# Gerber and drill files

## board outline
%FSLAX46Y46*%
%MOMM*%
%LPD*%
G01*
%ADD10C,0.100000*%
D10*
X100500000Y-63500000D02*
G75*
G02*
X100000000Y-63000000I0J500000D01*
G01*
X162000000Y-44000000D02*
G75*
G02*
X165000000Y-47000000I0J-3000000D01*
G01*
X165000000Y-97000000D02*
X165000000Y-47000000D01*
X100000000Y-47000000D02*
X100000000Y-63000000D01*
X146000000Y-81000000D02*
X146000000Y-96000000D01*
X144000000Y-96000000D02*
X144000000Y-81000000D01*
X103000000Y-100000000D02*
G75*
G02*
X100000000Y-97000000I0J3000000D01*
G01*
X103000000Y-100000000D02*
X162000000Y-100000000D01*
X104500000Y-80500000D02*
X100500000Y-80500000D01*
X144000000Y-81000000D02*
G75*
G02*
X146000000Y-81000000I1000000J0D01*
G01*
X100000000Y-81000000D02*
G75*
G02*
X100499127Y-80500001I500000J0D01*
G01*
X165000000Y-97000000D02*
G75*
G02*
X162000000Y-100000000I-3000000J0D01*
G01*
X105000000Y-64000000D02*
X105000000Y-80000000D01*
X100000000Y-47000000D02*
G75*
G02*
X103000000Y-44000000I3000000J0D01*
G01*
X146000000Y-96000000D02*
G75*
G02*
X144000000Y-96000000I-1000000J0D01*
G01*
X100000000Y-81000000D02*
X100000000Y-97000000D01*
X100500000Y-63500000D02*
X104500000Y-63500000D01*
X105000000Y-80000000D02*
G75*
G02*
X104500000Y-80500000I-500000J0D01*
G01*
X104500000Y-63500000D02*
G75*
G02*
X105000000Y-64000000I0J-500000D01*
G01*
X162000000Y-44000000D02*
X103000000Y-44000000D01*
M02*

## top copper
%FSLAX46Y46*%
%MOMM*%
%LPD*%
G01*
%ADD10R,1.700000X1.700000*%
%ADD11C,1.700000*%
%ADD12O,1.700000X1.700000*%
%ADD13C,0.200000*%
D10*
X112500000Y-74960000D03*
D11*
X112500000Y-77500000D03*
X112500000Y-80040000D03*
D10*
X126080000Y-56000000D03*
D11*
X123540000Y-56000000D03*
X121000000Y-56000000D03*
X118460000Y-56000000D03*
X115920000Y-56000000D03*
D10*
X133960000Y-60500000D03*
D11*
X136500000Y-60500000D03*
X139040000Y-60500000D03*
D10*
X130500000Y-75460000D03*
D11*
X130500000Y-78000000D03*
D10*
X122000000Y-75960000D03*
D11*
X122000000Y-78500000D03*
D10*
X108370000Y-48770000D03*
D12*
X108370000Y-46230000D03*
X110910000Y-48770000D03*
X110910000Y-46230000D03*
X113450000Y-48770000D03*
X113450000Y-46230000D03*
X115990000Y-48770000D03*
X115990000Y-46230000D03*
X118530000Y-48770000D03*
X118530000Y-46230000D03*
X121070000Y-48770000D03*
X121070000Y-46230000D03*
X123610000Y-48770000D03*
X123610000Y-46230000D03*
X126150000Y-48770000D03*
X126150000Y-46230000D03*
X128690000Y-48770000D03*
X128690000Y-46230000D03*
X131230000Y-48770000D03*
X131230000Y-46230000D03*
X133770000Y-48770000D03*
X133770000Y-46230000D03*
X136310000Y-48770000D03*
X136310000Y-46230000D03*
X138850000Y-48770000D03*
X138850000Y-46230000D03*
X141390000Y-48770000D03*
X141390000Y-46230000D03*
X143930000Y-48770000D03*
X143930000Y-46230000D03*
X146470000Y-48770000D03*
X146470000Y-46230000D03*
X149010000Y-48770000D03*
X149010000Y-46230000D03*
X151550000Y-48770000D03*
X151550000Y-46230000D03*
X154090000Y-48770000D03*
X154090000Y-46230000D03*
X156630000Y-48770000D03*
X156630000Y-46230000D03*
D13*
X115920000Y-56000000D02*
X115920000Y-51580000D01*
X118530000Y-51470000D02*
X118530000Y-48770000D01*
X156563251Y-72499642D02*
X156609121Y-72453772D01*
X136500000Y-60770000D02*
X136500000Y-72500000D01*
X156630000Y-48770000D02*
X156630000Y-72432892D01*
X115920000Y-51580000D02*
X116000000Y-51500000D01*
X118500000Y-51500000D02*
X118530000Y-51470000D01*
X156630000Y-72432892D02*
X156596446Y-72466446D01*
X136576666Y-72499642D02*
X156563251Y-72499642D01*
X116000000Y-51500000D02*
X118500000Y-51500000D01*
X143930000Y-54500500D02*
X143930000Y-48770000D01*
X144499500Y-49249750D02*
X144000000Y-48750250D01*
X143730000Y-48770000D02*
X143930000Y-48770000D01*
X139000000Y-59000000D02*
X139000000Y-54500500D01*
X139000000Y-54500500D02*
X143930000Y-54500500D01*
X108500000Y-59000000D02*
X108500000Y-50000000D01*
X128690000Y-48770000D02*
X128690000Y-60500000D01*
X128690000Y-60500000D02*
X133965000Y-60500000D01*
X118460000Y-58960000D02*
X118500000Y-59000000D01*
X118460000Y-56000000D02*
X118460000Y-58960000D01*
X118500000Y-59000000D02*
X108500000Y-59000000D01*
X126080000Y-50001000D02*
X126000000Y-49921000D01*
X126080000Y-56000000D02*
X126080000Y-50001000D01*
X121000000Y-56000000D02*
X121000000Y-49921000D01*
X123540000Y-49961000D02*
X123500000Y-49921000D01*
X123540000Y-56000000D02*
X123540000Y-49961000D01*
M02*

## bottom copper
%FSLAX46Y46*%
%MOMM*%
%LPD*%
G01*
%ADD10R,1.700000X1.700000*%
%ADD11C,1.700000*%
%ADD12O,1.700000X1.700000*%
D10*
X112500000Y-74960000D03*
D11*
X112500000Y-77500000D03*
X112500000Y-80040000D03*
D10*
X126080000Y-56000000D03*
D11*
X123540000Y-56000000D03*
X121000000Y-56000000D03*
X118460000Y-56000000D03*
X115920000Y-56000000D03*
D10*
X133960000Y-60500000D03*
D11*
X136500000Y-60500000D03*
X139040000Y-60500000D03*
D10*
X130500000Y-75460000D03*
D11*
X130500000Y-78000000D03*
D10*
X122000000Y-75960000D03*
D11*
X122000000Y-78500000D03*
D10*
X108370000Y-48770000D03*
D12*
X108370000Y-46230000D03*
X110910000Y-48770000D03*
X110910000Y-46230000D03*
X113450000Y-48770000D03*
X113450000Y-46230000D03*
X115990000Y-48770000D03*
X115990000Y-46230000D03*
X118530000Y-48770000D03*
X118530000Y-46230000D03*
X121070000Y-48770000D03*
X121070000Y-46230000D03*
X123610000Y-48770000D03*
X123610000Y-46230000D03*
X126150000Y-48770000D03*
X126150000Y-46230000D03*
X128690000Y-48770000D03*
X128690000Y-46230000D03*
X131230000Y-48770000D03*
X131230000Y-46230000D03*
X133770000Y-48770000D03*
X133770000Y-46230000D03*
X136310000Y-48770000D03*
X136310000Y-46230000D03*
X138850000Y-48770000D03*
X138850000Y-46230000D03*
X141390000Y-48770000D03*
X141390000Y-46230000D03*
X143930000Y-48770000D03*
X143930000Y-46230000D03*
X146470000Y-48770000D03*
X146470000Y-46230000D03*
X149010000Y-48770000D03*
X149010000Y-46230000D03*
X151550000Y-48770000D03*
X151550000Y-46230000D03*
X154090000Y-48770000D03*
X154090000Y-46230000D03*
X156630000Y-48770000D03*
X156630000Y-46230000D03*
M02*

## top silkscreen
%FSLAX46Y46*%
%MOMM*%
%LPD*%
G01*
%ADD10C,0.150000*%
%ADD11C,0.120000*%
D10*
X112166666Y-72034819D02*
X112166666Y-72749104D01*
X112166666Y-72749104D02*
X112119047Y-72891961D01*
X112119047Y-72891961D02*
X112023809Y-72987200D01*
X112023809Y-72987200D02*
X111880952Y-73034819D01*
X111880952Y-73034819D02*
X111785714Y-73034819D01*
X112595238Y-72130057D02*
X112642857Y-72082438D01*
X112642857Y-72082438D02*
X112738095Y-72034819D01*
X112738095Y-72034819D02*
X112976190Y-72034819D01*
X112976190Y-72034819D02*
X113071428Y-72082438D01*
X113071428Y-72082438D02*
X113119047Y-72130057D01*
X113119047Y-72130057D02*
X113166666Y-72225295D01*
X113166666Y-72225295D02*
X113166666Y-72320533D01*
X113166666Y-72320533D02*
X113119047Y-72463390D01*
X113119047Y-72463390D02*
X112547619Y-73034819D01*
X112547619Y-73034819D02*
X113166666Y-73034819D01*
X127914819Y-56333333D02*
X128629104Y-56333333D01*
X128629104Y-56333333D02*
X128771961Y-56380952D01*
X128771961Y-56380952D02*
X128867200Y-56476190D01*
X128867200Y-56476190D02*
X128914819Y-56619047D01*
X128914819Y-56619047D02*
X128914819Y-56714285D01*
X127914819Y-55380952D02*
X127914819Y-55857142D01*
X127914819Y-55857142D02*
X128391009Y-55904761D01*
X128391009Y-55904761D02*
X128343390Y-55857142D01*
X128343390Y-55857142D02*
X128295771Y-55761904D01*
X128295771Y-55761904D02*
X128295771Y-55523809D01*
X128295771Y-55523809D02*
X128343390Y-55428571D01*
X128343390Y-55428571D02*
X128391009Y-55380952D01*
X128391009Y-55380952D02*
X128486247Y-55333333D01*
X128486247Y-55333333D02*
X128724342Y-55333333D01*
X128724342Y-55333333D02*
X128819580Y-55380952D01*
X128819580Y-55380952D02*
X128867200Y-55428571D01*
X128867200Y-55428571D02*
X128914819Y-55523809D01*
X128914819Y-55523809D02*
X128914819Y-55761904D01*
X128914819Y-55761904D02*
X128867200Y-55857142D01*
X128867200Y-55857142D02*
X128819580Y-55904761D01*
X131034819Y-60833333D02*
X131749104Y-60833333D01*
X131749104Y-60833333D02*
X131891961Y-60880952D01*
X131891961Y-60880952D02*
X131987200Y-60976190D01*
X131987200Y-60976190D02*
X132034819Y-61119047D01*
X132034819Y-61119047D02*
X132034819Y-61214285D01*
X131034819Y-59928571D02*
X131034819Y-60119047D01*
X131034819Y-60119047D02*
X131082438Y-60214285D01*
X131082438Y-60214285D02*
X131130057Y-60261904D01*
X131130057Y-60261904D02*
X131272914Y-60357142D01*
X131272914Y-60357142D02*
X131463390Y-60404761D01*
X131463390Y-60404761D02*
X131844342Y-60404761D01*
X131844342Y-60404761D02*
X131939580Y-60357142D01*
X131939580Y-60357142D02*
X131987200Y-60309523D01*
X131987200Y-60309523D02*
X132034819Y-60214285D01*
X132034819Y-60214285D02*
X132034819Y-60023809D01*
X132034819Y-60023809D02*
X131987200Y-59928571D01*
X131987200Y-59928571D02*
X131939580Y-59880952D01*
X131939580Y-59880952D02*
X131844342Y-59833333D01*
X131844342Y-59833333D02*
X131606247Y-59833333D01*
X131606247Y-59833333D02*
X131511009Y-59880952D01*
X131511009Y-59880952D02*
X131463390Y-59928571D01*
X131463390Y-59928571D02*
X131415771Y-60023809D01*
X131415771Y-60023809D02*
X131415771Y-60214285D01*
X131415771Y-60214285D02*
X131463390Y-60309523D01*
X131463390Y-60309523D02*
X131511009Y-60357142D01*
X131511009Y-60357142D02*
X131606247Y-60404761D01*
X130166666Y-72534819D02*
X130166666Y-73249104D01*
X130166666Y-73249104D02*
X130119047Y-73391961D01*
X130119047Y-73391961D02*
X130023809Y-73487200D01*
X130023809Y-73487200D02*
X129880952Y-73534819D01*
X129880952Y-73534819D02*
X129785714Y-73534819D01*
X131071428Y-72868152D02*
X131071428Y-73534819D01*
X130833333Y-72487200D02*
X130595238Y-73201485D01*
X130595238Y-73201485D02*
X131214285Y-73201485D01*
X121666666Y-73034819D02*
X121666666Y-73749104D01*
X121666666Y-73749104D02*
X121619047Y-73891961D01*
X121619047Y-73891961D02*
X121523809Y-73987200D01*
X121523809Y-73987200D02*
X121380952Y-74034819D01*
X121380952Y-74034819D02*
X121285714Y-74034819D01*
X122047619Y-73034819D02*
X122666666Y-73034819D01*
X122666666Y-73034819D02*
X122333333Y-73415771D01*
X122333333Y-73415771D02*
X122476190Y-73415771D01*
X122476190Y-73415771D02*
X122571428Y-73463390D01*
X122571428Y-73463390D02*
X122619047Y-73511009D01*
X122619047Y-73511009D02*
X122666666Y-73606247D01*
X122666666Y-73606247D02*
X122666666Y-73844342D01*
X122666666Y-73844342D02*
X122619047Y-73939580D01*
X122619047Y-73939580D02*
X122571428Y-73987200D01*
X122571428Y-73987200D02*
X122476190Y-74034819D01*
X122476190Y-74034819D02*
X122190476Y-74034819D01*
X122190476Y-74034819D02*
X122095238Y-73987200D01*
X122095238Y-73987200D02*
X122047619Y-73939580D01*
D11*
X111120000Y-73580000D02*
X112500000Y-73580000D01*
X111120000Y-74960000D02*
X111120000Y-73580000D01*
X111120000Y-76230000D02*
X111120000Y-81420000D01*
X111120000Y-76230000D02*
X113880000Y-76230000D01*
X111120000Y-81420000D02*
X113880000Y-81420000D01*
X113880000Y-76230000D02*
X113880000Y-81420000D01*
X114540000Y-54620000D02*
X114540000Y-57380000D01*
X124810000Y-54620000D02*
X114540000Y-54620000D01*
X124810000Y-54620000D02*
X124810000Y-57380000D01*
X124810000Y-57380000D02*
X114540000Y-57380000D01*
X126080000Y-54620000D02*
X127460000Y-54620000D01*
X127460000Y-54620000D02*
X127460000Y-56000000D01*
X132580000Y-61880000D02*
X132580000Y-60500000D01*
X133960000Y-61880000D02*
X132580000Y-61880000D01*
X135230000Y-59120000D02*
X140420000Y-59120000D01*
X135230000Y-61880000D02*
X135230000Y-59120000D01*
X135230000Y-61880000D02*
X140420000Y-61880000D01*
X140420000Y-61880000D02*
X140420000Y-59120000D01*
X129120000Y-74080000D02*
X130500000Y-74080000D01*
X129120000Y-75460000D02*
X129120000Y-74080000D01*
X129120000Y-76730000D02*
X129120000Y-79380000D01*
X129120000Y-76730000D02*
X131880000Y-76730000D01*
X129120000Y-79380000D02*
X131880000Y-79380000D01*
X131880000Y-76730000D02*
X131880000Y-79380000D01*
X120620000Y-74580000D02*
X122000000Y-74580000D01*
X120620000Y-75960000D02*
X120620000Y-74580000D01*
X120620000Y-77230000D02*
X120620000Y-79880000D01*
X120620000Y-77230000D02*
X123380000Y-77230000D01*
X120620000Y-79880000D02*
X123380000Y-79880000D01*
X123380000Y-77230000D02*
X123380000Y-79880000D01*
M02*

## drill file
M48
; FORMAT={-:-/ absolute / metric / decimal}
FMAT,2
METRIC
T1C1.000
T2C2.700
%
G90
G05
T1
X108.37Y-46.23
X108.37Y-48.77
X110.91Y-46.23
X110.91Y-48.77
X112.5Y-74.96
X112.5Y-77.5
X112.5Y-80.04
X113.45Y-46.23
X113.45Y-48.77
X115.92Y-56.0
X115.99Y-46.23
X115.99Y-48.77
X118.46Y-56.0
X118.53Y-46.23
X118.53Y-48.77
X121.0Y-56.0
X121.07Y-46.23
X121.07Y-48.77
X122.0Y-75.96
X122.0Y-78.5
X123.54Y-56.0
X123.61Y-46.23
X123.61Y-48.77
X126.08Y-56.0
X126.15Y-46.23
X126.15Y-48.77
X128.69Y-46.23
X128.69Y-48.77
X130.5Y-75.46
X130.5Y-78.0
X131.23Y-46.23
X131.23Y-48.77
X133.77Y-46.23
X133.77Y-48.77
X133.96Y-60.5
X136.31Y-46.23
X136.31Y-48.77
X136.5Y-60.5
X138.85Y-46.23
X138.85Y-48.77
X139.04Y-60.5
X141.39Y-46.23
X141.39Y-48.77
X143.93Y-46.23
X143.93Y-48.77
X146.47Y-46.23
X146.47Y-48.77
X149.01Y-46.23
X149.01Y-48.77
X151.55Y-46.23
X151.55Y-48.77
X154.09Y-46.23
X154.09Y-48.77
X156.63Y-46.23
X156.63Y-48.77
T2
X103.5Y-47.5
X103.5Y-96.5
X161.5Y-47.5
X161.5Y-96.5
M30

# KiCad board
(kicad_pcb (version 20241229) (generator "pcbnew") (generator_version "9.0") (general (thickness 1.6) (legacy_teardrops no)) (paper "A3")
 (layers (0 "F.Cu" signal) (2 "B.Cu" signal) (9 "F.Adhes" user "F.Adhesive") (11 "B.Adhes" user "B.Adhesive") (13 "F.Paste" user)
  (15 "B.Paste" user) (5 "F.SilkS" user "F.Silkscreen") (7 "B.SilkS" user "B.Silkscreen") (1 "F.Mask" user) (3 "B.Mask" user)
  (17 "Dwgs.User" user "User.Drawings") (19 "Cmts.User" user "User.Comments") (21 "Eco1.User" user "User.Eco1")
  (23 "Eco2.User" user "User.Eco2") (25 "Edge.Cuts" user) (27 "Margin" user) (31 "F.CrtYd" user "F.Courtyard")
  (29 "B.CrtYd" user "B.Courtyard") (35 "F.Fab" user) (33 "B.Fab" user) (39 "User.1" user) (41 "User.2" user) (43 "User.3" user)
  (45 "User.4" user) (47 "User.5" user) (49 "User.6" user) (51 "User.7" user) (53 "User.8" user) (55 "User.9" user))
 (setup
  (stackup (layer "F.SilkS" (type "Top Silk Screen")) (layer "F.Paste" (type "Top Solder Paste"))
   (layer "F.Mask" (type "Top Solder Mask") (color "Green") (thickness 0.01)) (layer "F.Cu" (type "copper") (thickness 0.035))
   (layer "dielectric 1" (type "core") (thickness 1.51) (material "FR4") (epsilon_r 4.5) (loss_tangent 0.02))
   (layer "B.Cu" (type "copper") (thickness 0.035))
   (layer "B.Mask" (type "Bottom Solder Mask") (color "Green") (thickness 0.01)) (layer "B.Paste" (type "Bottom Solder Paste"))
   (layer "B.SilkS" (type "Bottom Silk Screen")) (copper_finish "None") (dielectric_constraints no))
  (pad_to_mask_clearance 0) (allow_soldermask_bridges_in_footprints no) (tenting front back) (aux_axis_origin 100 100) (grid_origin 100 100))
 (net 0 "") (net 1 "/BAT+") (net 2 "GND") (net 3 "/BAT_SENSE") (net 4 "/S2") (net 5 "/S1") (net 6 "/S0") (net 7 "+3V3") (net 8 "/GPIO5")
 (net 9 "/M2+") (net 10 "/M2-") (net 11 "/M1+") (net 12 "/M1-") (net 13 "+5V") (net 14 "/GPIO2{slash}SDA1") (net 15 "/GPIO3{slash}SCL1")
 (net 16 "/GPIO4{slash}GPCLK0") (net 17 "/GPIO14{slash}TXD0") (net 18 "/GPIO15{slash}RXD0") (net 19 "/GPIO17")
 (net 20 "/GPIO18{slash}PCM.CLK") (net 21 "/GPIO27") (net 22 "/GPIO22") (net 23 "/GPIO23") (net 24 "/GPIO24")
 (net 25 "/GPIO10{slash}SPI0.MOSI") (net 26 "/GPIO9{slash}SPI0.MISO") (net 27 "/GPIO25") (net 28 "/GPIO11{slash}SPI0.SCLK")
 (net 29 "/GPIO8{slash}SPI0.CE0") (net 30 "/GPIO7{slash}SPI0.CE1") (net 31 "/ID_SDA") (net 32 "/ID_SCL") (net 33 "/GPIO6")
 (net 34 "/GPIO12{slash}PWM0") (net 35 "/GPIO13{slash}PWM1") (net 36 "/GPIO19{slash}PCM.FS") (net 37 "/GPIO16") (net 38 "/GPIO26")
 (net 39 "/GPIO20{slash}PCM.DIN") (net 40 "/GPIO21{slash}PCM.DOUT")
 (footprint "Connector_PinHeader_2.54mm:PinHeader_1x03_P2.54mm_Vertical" (layer "F.Cu") (at 112.5 74.96)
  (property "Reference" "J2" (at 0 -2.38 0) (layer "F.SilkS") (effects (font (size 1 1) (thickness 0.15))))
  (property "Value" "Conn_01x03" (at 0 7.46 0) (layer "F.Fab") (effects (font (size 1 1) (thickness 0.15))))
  (fp_line (start -1.38 -1.38) (end 0 -1.38) (stroke (width 0.12) (type solid)) (layer "F.SilkS"))
  (fp_line (start -1.38 0) (end -1.38 -1.38) (stroke (width 0.12) (type solid)) (layer "F.SilkS"))
  (fp_line (start -1.38 1.27) (end -1.38 6.46) (stroke (width 0.12) (type solid)) (layer "F.SilkS"))
  (fp_line (start -1.38 1.27) (end 1.38 1.27) (stroke (width 0.12) (type solid)) (layer "F.SilkS"))
  (fp_line (start -1.38 6.46) (end 1.38 6.46) (stroke (width 0.12) (type solid)) (layer "F.SilkS"))
  (fp_line (start 1.38 1.27) (end 1.38 6.46) (stroke (width 0.12) (type solid)) (layer "F.SilkS"))
  (pad "1" thru_hole rect (at 0 0) (size 1.7 1.7) (drill 1) (layers "*.Cu" "*.Mask") (remove_unused_layers no) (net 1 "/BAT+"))
  (pad "2" thru_hole circle (at 0 2.54) (size 1.7 1.7) (drill 1) (layers "*.Cu" "*.Mask") (remove_unused_layers no) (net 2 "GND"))
  (pad "3" thru_hole circle (at 0 5.08) (size 1.7 1.7) (drill 1) (layers "*.Cu" "*.Mask") (remove_unused_layers no) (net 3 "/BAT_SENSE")))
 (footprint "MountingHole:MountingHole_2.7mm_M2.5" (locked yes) (layer "F.Cu") (at 161.5 47.5)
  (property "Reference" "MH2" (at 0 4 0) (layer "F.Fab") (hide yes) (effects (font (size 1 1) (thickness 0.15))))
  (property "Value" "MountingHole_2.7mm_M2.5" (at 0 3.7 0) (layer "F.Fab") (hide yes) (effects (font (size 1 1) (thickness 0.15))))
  (pad "" np_thru_hole circle (at 0 0) (size 2.7 2.7) (drill 2.7) (layers "*.Cu" "*.Mask")))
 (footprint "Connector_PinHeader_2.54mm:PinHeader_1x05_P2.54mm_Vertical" (layer "F.Cu") (at 126.08 56 -90)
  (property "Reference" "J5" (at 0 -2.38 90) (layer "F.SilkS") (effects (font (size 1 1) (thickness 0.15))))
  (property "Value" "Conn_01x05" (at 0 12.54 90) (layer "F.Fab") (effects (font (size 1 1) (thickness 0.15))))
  (fp_line (start -1.38 11.54) (end 1.38 11.54) (stroke (width 0.12) (type solid)) (layer "F.SilkS"))
  (fp_line (start -1.38 1.27) (end -1.38 11.54) (stroke (width 0.12) (type solid)) (layer "F.SilkS"))
  (fp_line (start -1.38 1.27) (end 1.38 1.27) (stroke (width 0.12) (type solid)) (layer "F.SilkS"))
  (fp_line (start 1.38 1.27) (end 1.38 11.54) (stroke (width 0.12) (type solid)) (layer "F.SilkS"))
  (fp_line (start -1.38 0) (end -1.38 -1.38) (stroke (width 0.12) (type solid)) (layer "F.SilkS"))
  (fp_line (start -1.38 -1.38) (end 0 -1.38) (stroke (width 0.12) (type solid)) (layer "F.SilkS"))
  (pad "1" thru_hole rect (at 0 0 270) (size 1.7 1.7) (drill 1) (layers "*.Cu" "*.Mask") (remove_unused_layers no) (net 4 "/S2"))
  (pad "2" thru_hole circle (at 0 2.54 270) (size 1.7 1.7) (drill 1) (layers "*.Cu" "*.Mask") (remove_unused_layers no) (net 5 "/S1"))
  (pad "3" thru_hole circle (at 0 5.08 270) (size 1.7 1.7) (drill 1) (layers "*.Cu" "*.Mask") (remove_unused_layers no) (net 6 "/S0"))
  (pad "4" thru_hole circle (at 0 7.62 270) (size 1.7 1.7) (drill 1) (layers "*.Cu" "*.Mask") (remove_unused_layers no) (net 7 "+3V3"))
  (pad "5" thru_hole circle (at 0 10.16 270) (size 1.7 1.7) (drill 1) (layers "*.Cu" "*.Mask") (remove_unused_layers no) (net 2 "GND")))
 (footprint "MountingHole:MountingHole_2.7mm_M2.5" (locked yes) (layer "F.Cu") (at 103.5 96.5)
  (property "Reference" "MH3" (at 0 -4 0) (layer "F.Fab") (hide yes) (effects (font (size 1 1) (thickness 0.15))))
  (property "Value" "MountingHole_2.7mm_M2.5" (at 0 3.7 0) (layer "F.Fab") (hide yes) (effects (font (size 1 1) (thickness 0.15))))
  (pad "" np_thru_hole circle (at 0 0) (size 2.7 2.7) (drill 2.7) (layers "*.Cu" "*.Mask")))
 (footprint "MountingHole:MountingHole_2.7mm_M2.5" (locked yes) (layer "F.Cu") (at 103.5 47.5)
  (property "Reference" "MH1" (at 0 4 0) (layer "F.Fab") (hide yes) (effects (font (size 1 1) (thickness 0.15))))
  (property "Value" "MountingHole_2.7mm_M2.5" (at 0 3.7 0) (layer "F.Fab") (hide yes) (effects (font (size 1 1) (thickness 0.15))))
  (pad "" np_thru_hole circle (at 0 0) (size 2.7 2.7) (drill 2.7) (layers "*.Cu" "*.Mask")))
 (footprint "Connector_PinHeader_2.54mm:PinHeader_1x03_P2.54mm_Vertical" (layer "F.Cu") (at 133.96 60.5 90)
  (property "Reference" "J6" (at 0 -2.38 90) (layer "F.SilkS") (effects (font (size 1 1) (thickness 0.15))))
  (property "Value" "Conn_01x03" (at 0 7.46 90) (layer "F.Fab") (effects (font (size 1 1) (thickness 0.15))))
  (fp_line (start -1.38 -1.38) (end 0 -1.38) (stroke (width 0.12) (type solid)) (layer "F.SilkS"))
  (fp_line (start -1.38 0) (end -1.38 -1.38) (stroke (width 0.12) (type solid)) (layer "F.SilkS"))
  (fp_line (start 1.38 1.27) (end 1.38 6.46) (stroke (width 0.12) (type solid)) (layer "F.SilkS"))
  (fp_line (start -1.38 1.27) (end 1.38 1.27) (stroke (width 0.12) (type solid)) (layer "F.SilkS"))
  (fp_line (start -1.38 1.27) (end -1.38 6.46) (stroke (width 0.12) (type solid)) (layer "F.SilkS"))
  (fp_line (start -1.38 6.46) (end 1.38 6.46) (stroke (width 0.12) (type solid)) (layer "F.SilkS"))
  (pad "1" thru_hole rect (at 0 0 90) (size 1.7 1.7) (drill 1) (layers "*.Cu" "*.Mask") (remove_unused_layers no) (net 7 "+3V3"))
  (pad "2" thru_hole circle (at 0 2.54 90) (size 1.7 1.7) (drill 1) (layers "*.Cu" "*.Mask") (remove_unused_layers no) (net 2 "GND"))
  (pad "3" thru_hole circle (at 0 5.08 90) (size 1.7 1.7) (drill 1) (layers "*.Cu" "*.Mask") (remove_unused_layers no) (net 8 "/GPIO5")))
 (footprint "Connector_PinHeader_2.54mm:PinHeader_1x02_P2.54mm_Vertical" (layer "F.Cu") (at 130.5 75.46)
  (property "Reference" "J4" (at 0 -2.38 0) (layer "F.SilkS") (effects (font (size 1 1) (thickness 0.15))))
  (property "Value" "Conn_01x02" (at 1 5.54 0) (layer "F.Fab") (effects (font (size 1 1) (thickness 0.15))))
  (fp_line (start -1.38 -1.38) (end 0 -1.38) (stroke (width 0.12) (type solid)) (layer "F.SilkS"))
  (fp_line (start -1.38 0) (end -1.38 -1.38) (stroke (width 0.12) (type solid)) (layer "F.SilkS"))
  (fp_line (start -1.38 1.27) (end -1.38 3.92) (stroke (width 0.12) (type solid)) (layer "F.SilkS"))
  (fp_line (start -1.38 1.27) (end 1.38 1.27) (stroke (width 0.12) (type solid)) (layer "F.SilkS"))
  (fp_line (start -1.38 3.92) (end 1.38 3.92) (stroke (width 0.12) (type solid)) (layer "F.SilkS"))
  (fp_line (start 1.38 1.27) (end 1.38 3.92) (stroke (width 0.12) (type solid)) (layer "F.SilkS"))
  (pad "1" thru_hole rect (at 0 0) (size 1.7 1.7) (drill 1) (layers "*.Cu" "*.Mask") (remove_unused_layers no) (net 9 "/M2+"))
  (pad "2" thru_hole circle (at 0 2.54) (size 1.7 1.7) (drill 1) (layers "*.Cu" "*.Mask") (remove_unused_layers no) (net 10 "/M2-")))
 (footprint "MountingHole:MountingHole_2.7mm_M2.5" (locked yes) (layer "F.Cu") (at 161.5 96.5)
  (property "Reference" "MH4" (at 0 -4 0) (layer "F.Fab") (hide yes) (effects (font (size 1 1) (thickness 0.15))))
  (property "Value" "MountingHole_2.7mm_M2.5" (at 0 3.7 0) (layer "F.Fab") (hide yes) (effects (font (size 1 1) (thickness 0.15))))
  (pad "" np_thru_hole circle (at 0 0) (size 2.7 2.7) (drill 2.7) (layers "*.Cu" "*.Mask")))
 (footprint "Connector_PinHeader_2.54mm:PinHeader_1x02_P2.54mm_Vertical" (layer "F.Cu") (at 122 75.96)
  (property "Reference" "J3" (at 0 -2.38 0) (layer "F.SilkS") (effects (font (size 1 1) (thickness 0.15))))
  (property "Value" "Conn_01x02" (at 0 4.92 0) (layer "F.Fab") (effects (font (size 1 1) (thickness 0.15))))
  (fp_line (start -1.38 -1.38) (end 0 -1.38) (stroke (width 0.12) (type solid)) (layer "F.SilkS"))
  (fp_line (start -1.38 0) (end -1.38 -1.38) (stroke (width 0.12) (type solid)) (layer "F.SilkS"))
  (fp_line (start -1.38 1.27) (end -1.38 3.92) (stroke (width 0.12) (type solid)) (layer "F.SilkS"))
  (fp_line (start -1.38 1.27) (end 1.38 1.27) (stroke (width 0.12) (type solid)) (layer "F.SilkS"))
  (fp_line (start -1.38 3.92) (end 1.38 3.92) (stroke (width 0.12) (type solid)) (layer "F.SilkS"))
  (fp_line (start 1.38 1.27) (end 1.38 3.92) (stroke (width 0.12) (type solid)) (layer "F.SilkS"))
  (pad "1" thru_hole rect (at 0 0) (size 1.7 1.7) (drill 1) (layers "*.Cu" "*.Mask") (remove_unused_layers no) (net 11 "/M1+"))
  (pad "2" thru_hole circle (at 0 2.54) (size 1.7 1.7) (drill 1) (layers "*.Cu" "*.Mask") (remove_unused_layers no) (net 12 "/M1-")))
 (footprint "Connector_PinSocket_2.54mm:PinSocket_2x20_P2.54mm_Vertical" (layer "B.Cu") (at 108.37 48.77 -90)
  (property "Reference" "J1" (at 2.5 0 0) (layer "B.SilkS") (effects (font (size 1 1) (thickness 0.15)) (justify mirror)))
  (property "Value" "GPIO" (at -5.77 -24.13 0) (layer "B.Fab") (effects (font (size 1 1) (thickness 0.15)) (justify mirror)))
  (pad "1" thru_hole rect (at 0 0 270) (size 1.7 1.7) (drill 1) (layers "*.Cu" "*.Mask") (remove_unused_layers no) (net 7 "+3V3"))
  (pad "2" thru_hole oval (at -2.54 0 270) (size 1.7 1.7) (drill 1) (layers "*.Cu" "*.Mask") (remove_unused_layers no) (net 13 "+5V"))
  (pad "3" thru_hole oval (at 0 -2.54 270) (size 1.7 1.7) (drill 1) (layers "*.Cu" "*.Mask") (remove_unused_layers no)
   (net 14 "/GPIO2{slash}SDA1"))
  (pad "4" thru_hole oval (at -2.54 -2.54 270) (size 1.7 1.7) (drill 1) (layers "*.Cu" "*.Mask") (remove_unused_layers no) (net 13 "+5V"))
  (pad "5" thru_hole oval (at 0 -5.08 270) (size 1.7 1.7) (drill 1) (layers "*.Cu" "*.Mask") (remove_unused_layers no)
   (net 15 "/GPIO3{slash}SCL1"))
  (pad "6" thru_hole oval (at -2.54 -5.08 270) (size 1.7 1.7) (drill 1) (layers "*.Cu" "*.Mask") (remove_unused_layers no) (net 2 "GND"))
  (pad "7" thru_hole oval (at 0 -7.62 270) (size 1.7 1.7) (drill 1) (layers "*.Cu" "*.Mask") (remove_unused_layers no)
   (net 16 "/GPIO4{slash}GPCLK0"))
  (pad "8" thru_hole oval (at -2.54 -7.62 270) (size 1.7 1.7) (drill 1) (layers "*.Cu" "*.Mask") (remove_unused_layers no)
   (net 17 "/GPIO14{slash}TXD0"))
  (pad "9" thru_hole oval (at 0 -10.16 270) (size 1.7 1.7) (drill 1) (layers "*.Cu" "*.Mask") (remove_unused_layers no) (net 2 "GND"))
  (pad "10" thru_hole oval (at -2.54 -10.16 270) (size 1.7 1.7) (drill 1) (layers "*.Cu" "*.Mask") (remove_unused_layers no)
   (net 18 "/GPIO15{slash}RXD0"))
  (pad "11" thru_hole oval (at 0 -12.7 270) (size 1.7 1.7) (drill 1) (layers "*.Cu" "*.Mask") (remove_unused_layers no) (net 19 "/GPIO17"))
  (pad "12" thru_hole oval (at -2.54 -12.7 270) (size 1.7 1.7) (drill 1) (layers "*.Cu" "*.Mask") (remove_unused_layers no)
   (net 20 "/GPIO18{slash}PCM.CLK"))
  (pad "13" thru_hole oval (at 0 -15.24 270) (size 1.7 1.7) (drill 1) (layers "*.Cu" "*.Mask") (remove_unused_layers no) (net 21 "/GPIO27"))
  (pad "14" thru_hole oval (at -2.54 -15.24 270) (size 1.7 1.7) (drill 1) (layers "*.Cu" "*.Mask") (remove_unused_layers no) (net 2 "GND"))
  (pad "15" thru_hole oval (at 0 -17.78 270) (size 1.7 1.7) (drill 1) (layers "*.Cu" "*.Mask") (remove_unused_layers no) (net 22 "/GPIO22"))
  (pad "16" thru_hole oval (at -2.54 -17.78 270) (size 1.7 1.7) (drill 1) (layers "*.Cu" "*.Mask") (remove_unused_layers no)
   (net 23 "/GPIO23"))
  (pad "17" thru_hole oval (at 0 -20.32 270) (size 1.7 1.7) (drill 1) (layers "*.Cu" "*.Mask") (remove_unused_layers no) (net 7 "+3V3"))
  (pad "18" thru_hole oval (at -2.54 -20.32 270) (size 1.7 1.7) (drill 1) (layers "*.Cu" "*.Mask") (remove_unused_layers no)
   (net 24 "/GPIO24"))
  (pad "19" thru_hole oval (at 0 -22.86 270) (size 1.7 1.7) (drill 1) (layers "*.Cu" "*.Mask") (remove_unused_layers no)
   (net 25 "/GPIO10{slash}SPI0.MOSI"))
  (pad "20" thru_hole oval (at -2.54 -22.86 270) (size 1.7 1.7) (drill 1) (layers "*.Cu" "*.Mask") (remove_unused_layers no) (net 2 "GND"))
  (pad "21" thru_hole oval (at 0 -25.4 270) (size 1.7 1.7) (drill 1) (layers "*.Cu" "*.Mask") (remove_unused_layers no)
   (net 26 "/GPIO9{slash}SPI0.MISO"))
  (pad "22" thru_hole oval (at -2.54 -25.4 270) (size 1.7 1.7) (drill 1) (layers "*.Cu" "*.Mask") (remove_unused_layers no)
   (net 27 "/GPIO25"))
  (pad "23" thru_hole oval (at 0 -27.94 270) (size 1.7 1.7) (drill 1) (layers "*.Cu" "*.Mask") (remove_unused_layers no)
   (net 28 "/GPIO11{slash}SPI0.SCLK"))
  (pad "24" thru_hole oval (at -2.54 -27.94 270) (size 1.7 1.7) (drill 1) (layers "*.Cu" "*.Mask") (remove_unused_layers no)
   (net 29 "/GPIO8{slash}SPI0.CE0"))
  (pad "25" thru_hole oval (at 0 -30.48 270) (size 1.7 1.7) (drill 1) (layers "*.Cu" "*.Mask") (remove_unused_layers no) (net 2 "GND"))
  (pad "26" thru_hole oval (at -2.54 -30.48 270) (size 1.7 1.7) (drill 1) (layers "*.Cu" "*.Mask") (remove_unused_layers no)
   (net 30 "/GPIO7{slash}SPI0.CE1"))
  (pad "27" thru_hole oval (at 0 -33.02 270) (size 1.7 1.7) (drill 1) (layers "*.Cu" "*.Mask") (remove_unused_layers no) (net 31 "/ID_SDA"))
  (pad "28" thru_hole oval (at -2.54 -33.02 270) (size 1.7 1.7) (drill 1) (layers "*.Cu" "*.Mask") (remove_unused_layers no)
   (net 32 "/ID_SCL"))
  (pad "29" thru_hole oval (at 0 -35.56 270) (size 1.7 1.7) (drill 1) (layers "*.Cu" "*.Mask") (remove_unused_layers no) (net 8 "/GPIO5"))
  (pad "30" thru_hole oval (at -2.54 -35.56 270) (size 1.7 1.7) (drill 1) (layers "*.Cu" "*.Mask") (remove_unused_layers no) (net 2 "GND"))
  (pad "31" thru_hole oval (at 0 -38.1 270) (size 1.7 1.7) (drill 1) (layers "*.Cu" "*.Mask") (remove_unused_layers no) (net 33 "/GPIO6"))
  (pad "32" thru_hole oval (at -2.54 -38.1 270) (size 1.7 1.7) (drill 1) (layers "*.Cu" "*.Mask") (remove_unused_layers no)
   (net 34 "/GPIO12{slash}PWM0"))
  (pad "33" thru_hole oval (at 0 -40.64 270) (size 1.7 1.7) (drill 1) (layers "*.Cu" "*.Mask") (remove_unused_layers no)
   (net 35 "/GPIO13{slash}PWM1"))
  (pad "34" thru_hole oval (at -2.54 -40.64 270) (size 1.7 1.7) (drill 1) (layers "*.Cu" "*.Mask") (remove_unused_layers no) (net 2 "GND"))
  (pad "35" thru_hole oval (at 0 -43.18 270) (size 1.7 1.7) (drill 1) (layers "*.Cu" "*.Mask") (remove_unused_layers no)
   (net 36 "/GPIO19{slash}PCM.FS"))
  (pad "36" thru_hole oval (at -2.54 -43.18 270) (size 1.7 1.7) (drill 1) (layers "*.Cu" "*.Mask") (remove_unused_layers no)
   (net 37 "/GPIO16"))
  (pad "37" thru_hole oval (at 0 -45.72 270) (size 1.7 1.7) (drill 1) (layers "*.Cu" "*.Mask") (remove_unused_layers no) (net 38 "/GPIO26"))
  (pad "38" thru_hole oval (at -2.54 -45.72 270) (size 1.7 1.7) (drill 1) (layers "*.Cu" "*.Mask") (remove_unused_layers no)
   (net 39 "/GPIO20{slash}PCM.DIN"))
  (pad "39" thru_hole oval (at 0 -48.26 270) (size 1.7 1.7) (drill 1) (layers "*.Cu" "*.Mask") (remove_unused_layers no) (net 2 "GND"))
  (pad "40" thru_hole oval (at -2.54 -48.26 270) (size 1.7 1.7) (drill 1) (layers "*.Cu" "*.Mask") (remove_unused_layers no)
   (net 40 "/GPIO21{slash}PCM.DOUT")))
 (gr_arc (start 100.5 63.5) (mid 100.146447 63.353553) (end 100 63) (stroke (width 0.1) (type solid)) (layer "Edge.Cuts"))
 (gr_arc (start 162 44) (mid 164.12132 44.87868) (end 165 47) (stroke (width 0.1) (type solid)) (layer "Edge.Cuts"))
 (gr_line (start 165 97) (end 165 47) (stroke (width 0.1) (type solid)) (layer "Edge.Cuts"))
 (gr_line (start 100 47) (end 100 63) (stroke (width 0.1) (type solid)) (layer "Edge.Cuts"))
 (gr_line (start 146 81) (end 146 96) (stroke (width 0.1) (type solid)) (layer "Edge.Cuts"))
 (gr_line (start 144 96) (end 144 81) (stroke (width 0.1) (type solid)) (layer "Edge.Cuts"))
 (gr_arc (start 103 100) (mid 100.87868 99.12132) (end 100 97) (stroke (width 0.1) (type solid)) (layer "Edge.Cuts"))
 (gr_line (start 103 100) (end 162 100) (stroke (width 0.1) (type solid)) (layer "Edge.Cuts"))
 (gr_line (start 104.5 80.5) (end 100.5 80.5) (stroke (width 0.1) (type solid)) (layer "Edge.Cuts"))
 (gr_arc (start 144 81) (mid 145 80) (end 146 81) (stroke (width 0.1) (type solid)) (layer "Edge.Cuts"))
 (gr_arc (start 100 81) (mid 100.146138 80.646755) (end 100.499127 80.500001) (stroke (width 0.1) (type solid)) (layer "Edge.Cuts"))
 (gr_arc (start 165 97) (mid 164.12132 99.12132) (end 162 100) (stroke (width 0.1) (type solid)) (layer "Edge.Cuts"))
 (gr_line (start 105 64) (end 105 80) (stroke (width 0.1) (type solid)) (layer "Edge.Cuts"))
 (gr_arc (start 100 47) (mid 100.87868 44.87868) (end 103 44) (stroke (width 0.1) (type solid)) (layer "Edge.Cuts"))
 (gr_arc (start 146 96) (mid 145 97) (end 144 96) (stroke (width 0.1) (type solid)) (layer "Edge.Cuts"))
 (gr_line (start 100 81) (end 100 97) (stroke (width 0.1) (type solid)) (layer "Edge.Cuts"))
 (gr_line (start 100.5 63.5) (end 104.5 63.5) (stroke (width 0.1) (type solid)) (layer "Edge.Cuts"))
 (gr_arc (start 105 80) (mid 104.853553 80.353553) (end 104.5 80.5) (stroke (width 0.1) (type solid)) (layer "Edge.Cuts"))
 (gr_arc (start 104.5 63.5) (mid 104.853553 63.646447) (end 105 64) (stroke (width 0.1) (type solid)) (layer "Edge.Cuts"))
 (gr_line (start 162 44) (end 103 44) (stroke (width 0.1) (type solid)) (layer "Edge.Cuts"))
 (segment (start 115.92 56) (end 115.92 51.58) (width 0.2) (layer "F.Cu") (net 2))
 (segment (start 118.53 51.47) (end 118.53 48.77) (width 0.2) (layer "F.Cu") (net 2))
 (segment (start 156.563251 72.499642) (end 156.609121 72.453772) (width 0.2) (layer "F.Cu") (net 2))
 (segment (start 136.5 60.77) (end 136.5 72.5) (width 0.2) (layer "F.Cu") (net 2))
 (segment (start 156.63 48.77) (end 156.63 72.432892) (width 0.2) (layer "F.Cu") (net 2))
 (segment (start 115.92 51.58) (end 116 51.5) (width 0.2) (layer "F.Cu") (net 2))
 (segment (start 118.5 51.5) (end 118.53 51.47) (width 0.2) (layer "F.Cu") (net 2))
 (segment (start 156.63 72.432892) (end 156.596446 72.466446) (width 0.2) (layer "F.Cu") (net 2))
 (segment (start 136.576666 72.499642) (end 156.563251 72.499642) (width 0.2) (layer "F.Cu") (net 2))
 (segment (start 116 51.5) (end 118.5 51.5) (width 0.2) (layer "F.Cu") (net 2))
 (segment (start 143.93 54.5005) (end 143.93 48.77) (width 0.2) (layer "F.Cu") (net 8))
 (segment (start 144.4995 49.24975) (end 144 48.75025) (width 0.2) (layer "F.Cu") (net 8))
 (segment (start 143.73 48.77) (end 143.93 48.77) (width 0.2) (layer "F.Cu") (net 8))
 (segment (start 139 59) (end 139 54.5005) (width 0.2) (layer "F.Cu") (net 8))
 (segment (start 139 54.5005) (end 143.93 54.5005) (width 0.2) (layer "F.Cu") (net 8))
 (segment (start 108.5 59) (end 108.5 50) (width 0.2) (layer "F.Cu") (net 7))
 (segment (start 128.69 48.77) (end 128.69 60.5) (width 0.2) (layer "F.Cu") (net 7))
 (segment (start 128.69 60.5) (end 133.965 60.5) (width 0.2) (layer "F.Cu") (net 7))
 (segment (start 118.46 58.96) (end 118.5 59) (width 0.2) (layer "F.Cu") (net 7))
 (segment (start 118.46 56) (end 118.46 58.96) (width 0.2) (layer "F.Cu") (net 7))
 (segment (start 118.5 59) (end 108.5 59) (width 0.2) (layer "F.Cu") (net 7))
 (segment (start 126.08 50.001) (end 126 49.921) (width 0.2) (layer "F.Cu") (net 4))
 (segment (start 126.08 56) (end 126.08 50.001) (width 0.2) (layer "F.Cu") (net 4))
 (segment (start 121 56) (end 121 49.921) (width 0.2) (layer "F.Cu") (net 6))
 (segment (start 123.54 49.961) (end 123.5 49.921) (width 0.2) (layer "F.Cu") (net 5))
 (segment (start 123.54 56) (end 123.54 49.961) (width 0.2) (layer "F.Cu") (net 5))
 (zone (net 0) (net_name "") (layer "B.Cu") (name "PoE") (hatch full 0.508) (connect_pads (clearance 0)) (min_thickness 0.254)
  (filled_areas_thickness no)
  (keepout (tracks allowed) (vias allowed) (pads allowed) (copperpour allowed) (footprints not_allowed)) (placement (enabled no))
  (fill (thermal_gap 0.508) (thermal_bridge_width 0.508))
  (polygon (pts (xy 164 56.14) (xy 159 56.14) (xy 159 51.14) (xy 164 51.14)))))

